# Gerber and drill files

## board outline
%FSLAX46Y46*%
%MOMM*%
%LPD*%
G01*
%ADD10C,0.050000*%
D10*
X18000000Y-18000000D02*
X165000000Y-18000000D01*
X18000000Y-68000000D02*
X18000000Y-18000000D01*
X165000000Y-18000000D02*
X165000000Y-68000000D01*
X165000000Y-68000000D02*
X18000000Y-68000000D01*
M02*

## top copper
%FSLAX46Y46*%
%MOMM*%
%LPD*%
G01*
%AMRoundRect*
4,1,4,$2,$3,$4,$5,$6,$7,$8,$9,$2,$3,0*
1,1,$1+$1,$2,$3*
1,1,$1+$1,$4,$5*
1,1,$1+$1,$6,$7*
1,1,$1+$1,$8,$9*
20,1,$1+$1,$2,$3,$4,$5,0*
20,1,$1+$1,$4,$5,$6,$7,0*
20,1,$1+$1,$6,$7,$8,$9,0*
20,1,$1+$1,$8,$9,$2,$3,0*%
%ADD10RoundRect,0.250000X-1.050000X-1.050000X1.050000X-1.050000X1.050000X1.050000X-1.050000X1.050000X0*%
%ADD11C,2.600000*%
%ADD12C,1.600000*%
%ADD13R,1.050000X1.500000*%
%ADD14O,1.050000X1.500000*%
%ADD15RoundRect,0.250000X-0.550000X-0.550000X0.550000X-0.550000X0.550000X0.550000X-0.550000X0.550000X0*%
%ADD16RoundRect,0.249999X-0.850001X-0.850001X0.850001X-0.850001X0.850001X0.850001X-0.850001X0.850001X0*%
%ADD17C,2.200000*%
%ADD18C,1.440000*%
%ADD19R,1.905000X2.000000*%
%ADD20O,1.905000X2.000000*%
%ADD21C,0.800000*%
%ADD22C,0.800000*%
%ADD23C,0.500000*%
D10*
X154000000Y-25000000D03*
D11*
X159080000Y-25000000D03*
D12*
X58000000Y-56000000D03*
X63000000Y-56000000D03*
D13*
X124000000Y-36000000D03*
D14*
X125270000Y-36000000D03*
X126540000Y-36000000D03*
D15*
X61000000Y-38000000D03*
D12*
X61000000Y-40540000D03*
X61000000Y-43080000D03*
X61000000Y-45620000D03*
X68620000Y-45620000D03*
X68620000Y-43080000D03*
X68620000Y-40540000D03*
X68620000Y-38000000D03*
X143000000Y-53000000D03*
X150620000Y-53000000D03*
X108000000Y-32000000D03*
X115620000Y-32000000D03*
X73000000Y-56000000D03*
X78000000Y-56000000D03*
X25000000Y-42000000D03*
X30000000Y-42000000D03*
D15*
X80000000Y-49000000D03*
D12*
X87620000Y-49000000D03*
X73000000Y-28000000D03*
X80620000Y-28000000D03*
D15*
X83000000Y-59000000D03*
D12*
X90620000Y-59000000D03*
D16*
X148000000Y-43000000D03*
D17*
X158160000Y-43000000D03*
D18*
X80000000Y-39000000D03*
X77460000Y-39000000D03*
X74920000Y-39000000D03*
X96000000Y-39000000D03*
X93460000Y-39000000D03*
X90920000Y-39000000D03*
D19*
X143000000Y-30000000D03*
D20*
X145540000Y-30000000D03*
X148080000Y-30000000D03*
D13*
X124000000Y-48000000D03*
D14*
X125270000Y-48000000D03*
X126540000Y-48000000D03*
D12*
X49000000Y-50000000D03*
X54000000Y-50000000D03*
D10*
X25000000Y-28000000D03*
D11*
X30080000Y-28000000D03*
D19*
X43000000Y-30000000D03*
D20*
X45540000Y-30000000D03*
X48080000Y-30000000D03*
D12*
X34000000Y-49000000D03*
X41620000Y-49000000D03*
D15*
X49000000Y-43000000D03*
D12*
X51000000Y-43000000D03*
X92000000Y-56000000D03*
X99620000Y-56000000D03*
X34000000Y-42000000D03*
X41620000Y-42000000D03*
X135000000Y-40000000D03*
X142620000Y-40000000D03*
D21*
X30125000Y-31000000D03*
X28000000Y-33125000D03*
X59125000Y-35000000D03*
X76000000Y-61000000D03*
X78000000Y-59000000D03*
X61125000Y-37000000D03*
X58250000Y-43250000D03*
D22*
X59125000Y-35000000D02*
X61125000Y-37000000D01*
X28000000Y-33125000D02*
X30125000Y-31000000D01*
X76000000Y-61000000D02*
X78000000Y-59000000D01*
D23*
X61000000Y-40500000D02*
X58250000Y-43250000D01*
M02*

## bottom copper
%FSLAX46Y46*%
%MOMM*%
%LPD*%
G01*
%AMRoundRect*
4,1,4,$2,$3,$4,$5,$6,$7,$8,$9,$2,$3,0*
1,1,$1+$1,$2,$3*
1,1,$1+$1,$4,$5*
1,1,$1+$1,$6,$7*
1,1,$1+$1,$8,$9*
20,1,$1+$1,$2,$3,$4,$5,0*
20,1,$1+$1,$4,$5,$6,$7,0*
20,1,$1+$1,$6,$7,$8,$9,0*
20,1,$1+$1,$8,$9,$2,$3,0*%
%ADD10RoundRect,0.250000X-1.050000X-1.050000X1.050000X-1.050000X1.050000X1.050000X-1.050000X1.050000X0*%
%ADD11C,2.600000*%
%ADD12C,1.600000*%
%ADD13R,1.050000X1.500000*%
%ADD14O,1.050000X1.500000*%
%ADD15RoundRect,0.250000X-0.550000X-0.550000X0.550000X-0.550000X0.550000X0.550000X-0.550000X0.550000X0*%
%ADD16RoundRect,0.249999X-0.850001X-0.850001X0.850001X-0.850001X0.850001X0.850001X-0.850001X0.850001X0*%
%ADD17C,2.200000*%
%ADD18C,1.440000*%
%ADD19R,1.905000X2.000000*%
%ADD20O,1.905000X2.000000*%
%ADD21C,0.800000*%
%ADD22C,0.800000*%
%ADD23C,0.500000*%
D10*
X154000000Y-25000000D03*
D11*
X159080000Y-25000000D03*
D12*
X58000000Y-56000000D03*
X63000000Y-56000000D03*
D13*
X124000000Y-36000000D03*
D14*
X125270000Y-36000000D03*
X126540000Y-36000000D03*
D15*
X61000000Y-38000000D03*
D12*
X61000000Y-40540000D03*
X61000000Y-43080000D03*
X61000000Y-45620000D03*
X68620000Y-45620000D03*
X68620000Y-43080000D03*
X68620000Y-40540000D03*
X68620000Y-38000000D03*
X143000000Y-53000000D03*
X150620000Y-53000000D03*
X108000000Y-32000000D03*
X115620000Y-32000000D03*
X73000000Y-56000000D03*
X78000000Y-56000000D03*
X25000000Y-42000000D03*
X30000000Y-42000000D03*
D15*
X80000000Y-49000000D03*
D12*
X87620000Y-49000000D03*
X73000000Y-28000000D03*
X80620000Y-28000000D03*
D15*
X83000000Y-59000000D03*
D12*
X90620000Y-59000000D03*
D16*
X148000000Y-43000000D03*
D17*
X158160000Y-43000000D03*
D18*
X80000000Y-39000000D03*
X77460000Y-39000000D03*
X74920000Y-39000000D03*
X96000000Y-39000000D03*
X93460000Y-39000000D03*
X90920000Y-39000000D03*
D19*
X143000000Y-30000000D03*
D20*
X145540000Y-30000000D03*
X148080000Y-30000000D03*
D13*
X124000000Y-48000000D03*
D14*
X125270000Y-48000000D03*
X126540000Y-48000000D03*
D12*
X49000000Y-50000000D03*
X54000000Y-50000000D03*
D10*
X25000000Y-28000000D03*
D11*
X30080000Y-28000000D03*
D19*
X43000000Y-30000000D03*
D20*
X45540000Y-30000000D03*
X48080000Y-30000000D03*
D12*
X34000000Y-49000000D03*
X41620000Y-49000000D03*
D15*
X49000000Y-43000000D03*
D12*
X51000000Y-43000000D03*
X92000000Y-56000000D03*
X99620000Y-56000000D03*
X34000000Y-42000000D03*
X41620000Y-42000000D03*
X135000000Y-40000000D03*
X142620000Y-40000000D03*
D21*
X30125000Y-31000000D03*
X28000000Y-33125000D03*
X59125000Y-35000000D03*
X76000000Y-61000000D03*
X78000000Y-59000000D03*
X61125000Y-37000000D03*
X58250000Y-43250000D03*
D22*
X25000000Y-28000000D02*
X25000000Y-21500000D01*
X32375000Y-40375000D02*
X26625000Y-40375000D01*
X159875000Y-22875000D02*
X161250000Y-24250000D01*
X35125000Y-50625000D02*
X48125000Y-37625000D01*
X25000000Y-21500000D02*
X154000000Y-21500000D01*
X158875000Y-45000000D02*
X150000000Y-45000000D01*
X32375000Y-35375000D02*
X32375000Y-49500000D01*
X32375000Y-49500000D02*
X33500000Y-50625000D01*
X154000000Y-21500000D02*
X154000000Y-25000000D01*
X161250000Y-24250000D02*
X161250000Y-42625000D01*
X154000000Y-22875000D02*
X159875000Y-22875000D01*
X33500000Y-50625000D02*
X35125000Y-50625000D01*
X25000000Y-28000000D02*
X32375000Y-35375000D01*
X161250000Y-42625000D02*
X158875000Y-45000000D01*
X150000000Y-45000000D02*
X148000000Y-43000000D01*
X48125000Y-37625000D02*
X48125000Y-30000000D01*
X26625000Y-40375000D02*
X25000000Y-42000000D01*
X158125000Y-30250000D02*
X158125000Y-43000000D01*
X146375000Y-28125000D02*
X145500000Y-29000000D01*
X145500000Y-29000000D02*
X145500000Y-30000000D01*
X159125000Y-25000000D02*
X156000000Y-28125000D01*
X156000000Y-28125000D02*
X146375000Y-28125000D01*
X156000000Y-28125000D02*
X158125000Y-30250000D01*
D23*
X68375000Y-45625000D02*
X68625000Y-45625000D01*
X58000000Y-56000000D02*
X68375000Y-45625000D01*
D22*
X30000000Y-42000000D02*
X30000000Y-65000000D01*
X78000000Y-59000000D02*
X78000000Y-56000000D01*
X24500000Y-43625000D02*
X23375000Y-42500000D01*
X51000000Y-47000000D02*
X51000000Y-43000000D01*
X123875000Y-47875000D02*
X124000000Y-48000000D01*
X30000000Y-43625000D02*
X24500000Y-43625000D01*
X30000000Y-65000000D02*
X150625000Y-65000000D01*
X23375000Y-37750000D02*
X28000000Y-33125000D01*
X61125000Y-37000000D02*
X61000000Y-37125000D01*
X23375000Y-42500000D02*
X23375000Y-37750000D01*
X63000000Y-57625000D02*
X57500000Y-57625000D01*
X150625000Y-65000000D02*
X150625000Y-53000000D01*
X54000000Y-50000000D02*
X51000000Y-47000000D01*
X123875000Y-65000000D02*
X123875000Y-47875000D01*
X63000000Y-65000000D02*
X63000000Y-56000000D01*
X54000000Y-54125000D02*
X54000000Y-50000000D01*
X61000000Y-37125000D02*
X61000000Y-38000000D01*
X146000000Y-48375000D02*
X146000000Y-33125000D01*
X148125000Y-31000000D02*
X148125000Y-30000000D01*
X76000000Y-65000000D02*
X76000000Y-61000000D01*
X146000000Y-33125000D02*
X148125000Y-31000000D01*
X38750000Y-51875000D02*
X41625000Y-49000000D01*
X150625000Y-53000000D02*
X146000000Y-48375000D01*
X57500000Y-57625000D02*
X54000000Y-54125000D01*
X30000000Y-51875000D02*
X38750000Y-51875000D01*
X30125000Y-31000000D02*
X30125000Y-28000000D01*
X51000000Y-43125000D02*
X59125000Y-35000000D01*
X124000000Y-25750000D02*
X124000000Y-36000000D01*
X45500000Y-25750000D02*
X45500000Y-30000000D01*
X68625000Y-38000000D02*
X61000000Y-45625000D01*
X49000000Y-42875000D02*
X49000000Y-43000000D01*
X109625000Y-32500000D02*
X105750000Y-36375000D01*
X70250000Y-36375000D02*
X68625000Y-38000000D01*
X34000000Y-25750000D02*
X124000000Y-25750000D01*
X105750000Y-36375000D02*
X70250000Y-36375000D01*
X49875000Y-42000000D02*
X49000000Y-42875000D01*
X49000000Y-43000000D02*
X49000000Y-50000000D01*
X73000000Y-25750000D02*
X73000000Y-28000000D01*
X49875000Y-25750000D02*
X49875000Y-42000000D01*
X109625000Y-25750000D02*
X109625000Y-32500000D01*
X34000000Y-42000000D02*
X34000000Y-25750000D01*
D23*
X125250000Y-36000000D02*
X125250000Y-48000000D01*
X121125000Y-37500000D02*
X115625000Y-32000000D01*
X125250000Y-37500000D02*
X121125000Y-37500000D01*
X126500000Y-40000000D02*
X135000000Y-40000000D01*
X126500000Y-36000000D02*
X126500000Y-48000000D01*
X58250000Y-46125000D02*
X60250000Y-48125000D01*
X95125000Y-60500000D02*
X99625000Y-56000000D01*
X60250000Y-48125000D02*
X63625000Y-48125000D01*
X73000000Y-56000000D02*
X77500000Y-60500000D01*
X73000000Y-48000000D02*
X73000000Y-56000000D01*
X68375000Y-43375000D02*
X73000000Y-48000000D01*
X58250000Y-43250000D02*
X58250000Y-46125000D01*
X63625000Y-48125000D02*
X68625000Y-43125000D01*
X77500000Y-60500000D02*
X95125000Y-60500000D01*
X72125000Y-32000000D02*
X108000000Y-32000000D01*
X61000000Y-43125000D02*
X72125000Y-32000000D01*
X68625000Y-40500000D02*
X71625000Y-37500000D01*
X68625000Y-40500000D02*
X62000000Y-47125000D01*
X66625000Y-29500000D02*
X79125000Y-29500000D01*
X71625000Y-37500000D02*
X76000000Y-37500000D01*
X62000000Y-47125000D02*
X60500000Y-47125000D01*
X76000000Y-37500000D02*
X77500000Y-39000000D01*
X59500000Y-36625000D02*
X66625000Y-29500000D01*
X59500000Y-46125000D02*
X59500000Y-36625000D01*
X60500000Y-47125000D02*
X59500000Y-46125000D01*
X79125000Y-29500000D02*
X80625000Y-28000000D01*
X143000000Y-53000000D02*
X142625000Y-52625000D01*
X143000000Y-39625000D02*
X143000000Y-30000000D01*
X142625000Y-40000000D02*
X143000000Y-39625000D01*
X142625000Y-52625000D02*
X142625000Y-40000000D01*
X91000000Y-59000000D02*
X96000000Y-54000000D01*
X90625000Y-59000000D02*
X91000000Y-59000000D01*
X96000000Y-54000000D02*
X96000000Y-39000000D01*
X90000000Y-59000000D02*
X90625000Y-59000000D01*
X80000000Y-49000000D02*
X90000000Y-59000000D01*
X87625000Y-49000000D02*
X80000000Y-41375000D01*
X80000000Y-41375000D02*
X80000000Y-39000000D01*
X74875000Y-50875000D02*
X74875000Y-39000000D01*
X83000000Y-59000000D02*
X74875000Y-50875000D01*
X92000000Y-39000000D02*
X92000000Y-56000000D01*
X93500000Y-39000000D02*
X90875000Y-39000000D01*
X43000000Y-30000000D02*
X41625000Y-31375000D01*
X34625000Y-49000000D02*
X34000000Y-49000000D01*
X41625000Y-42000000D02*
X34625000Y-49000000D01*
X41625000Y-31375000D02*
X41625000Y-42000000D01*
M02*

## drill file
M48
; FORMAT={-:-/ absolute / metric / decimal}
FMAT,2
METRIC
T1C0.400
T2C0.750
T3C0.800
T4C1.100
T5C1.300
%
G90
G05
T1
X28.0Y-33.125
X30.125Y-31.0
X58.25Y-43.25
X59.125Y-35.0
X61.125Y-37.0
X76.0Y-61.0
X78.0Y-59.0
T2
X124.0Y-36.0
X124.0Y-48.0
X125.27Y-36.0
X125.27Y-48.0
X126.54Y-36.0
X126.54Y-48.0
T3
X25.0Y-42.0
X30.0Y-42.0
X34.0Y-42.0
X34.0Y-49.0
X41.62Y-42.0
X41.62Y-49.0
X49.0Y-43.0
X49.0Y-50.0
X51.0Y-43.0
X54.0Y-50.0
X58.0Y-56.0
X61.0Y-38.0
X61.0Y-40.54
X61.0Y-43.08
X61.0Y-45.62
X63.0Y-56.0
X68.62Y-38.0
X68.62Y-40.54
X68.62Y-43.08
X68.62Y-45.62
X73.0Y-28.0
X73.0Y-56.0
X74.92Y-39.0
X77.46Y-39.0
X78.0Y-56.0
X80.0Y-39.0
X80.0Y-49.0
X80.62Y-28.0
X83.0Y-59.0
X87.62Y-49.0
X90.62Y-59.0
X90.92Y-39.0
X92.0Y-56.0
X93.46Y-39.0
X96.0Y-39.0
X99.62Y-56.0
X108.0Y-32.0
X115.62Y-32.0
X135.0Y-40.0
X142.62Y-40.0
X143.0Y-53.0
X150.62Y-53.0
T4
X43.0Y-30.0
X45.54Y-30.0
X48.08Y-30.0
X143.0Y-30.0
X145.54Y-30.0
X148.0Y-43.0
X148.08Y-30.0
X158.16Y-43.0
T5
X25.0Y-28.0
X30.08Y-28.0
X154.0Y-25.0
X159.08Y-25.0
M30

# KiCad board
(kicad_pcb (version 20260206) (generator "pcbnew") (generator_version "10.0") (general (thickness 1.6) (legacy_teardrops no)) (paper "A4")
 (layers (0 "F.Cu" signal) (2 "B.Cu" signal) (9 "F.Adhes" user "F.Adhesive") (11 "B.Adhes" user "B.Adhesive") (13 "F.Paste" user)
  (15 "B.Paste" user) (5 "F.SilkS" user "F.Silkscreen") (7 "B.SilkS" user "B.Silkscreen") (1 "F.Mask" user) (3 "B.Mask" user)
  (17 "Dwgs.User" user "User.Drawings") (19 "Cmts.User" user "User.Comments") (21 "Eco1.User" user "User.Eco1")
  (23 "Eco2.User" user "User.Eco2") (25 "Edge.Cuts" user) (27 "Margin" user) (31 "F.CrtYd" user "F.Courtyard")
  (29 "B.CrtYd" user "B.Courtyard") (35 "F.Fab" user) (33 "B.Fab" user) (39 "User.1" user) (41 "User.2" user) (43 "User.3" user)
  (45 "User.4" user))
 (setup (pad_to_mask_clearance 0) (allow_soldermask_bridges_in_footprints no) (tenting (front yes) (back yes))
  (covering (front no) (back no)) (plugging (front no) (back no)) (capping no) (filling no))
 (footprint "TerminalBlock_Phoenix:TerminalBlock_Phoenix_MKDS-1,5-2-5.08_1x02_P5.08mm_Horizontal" (layer "F.Cu") (at 154 25)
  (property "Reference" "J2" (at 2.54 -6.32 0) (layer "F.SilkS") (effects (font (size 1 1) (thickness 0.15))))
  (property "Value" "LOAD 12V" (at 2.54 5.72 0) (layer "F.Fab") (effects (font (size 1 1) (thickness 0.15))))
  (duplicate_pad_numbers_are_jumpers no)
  (pad "1" thru_hole roundrect (at 0 0) (size 2.6 2.6) (drill 1.3) (layers "*.Cu" "*.Mask") (remove_unused_layers no)
   (roundrect_rratio 0.096154) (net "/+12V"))
  (pad "2" thru_hole circle (at 5.08 0) (size 2.6 2.6) (drill 1.3) (layers "*.Cu" "*.Mask") (remove_unused_layers no) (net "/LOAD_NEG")))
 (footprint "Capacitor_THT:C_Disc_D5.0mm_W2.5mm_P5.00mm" (layer "F.Cu") (at 58 56)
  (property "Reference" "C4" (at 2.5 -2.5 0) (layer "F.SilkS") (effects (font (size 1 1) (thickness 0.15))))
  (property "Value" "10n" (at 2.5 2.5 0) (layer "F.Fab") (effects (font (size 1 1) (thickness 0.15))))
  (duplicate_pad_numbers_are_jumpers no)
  (pad "1" thru_hole circle (at 0 0) (size 1.6 1.6) (drill 0.8) (layers "*.Cu" "*.Mask") (remove_unused_layers no) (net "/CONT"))
  (pad "2" thru_hole circle (at 5 0) (size 1.6 1.6) (drill 0.8) (layers "*.Cu" "*.Mask") (remove_unused_layers no) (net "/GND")))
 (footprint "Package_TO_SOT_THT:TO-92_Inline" (layer "F.Cu") (at 124 36)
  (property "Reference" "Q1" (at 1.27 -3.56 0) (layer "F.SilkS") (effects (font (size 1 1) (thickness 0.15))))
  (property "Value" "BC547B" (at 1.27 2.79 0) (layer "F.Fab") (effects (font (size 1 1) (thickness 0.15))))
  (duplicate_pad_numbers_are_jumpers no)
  (pad "1" thru_hole rect (at 0 0) (size 1.05 1.5) (drill 0.75) (layers "*.Cu" "*.Mask") (remove_unused_layers no) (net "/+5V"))
  (pad "2" thru_hole oval (at 1.27 0) (size 1.05 1.5) (drill 0.75) (layers "*.Cu" "*.Mask") (remove_unused_layers no) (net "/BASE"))
  (pad "3" thru_hole oval (at 2.54 0) (size 1.05 1.5) (drill 0.75) (layers "*.Cu" "*.Mask") (remove_unused_layers no) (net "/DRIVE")))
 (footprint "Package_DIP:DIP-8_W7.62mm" (layer "F.Cu") (at 61 38)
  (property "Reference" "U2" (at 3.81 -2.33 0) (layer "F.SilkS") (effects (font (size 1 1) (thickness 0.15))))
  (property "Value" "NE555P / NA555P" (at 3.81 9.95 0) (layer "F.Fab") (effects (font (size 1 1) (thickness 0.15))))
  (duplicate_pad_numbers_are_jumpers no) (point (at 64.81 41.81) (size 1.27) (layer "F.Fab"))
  (pad "1" thru_hole roundrect (at 0 0) (size 1.6 1.6) (drill 0.8) (layers "*.Cu" "*.Mask") (remove_unused_layers no)
   (roundrect_rratio 0.15625) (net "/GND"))
  (pad "2" thru_hole circle (at 0 2.54) (size 1.6 1.6) (drill 0.8) (layers "*.Cu" "*.Mask") (remove_unused_layers no) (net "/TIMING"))
  (pad "3" thru_hole circle (at 0 5.08) (size 1.6 1.6) (drill 0.8) (layers "*.Cu" "*.Mask") (remove_unused_layers no) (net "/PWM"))
  (pad "4" thru_hole circle (at 0 7.62) (size 1.6 1.6) (drill 0.8) (layers "*.Cu" "*.Mask") (remove_unused_layers no) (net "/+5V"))
  (pad "5" thru_hole circle (at 7.62 7.62) (size 1.6 1.6) (drill 0.8) (layers "*.Cu" "*.Mask") (remove_unused_layers no) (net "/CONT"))
  (pad "6" thru_hole circle (at 7.62 5.08) (size 1.6 1.6) (drill 0.8) (layers "*.Cu" "*.Mask") (remove_unused_layers no) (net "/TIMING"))
  (pad "7" thru_hole circle (at 7.62 2.54) (size 1.6 1.6) (drill 0.8) (layers "*.Cu" "*.Mask") (remove_unused_layers no) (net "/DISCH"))
  (pad "8" thru_hole circle (at 7.62 0) (size 1.6 1.6) (drill 0.8) (layers "*.Cu" "*.Mask") (remove_unused_layers no) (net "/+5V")))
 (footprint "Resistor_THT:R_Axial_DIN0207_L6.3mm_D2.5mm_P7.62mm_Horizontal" (layer "F.Cu") (at 143 53)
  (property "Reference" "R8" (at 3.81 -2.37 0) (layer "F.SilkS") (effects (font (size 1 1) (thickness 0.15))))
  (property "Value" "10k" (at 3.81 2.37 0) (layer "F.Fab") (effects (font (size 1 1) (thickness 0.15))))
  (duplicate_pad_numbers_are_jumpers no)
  (pad "1" thru_hole circle (at 0 0) (size 1.6 1.6) (drill 0.8) (layers "*.Cu" "*.Mask") (remove_unused_layers no) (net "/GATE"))
  (pad "2" thru_hole circle (at 7.62 0) (size 1.6 1.6) (drill 0.8) (layers "*.Cu" "*.Mask") (remove_unused_layers no) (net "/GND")))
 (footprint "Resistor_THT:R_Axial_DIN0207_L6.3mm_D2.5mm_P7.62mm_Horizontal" (layer "F.Cu") (at 108 32)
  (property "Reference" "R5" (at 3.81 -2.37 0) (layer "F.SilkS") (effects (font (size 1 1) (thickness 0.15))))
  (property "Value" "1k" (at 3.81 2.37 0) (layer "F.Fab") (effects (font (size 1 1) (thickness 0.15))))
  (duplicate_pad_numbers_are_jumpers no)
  (pad "1" thru_hole circle (at 0 0) (size 1.6 1.6) (drill 0.8) (layers "*.Cu" "*.Mask") (remove_unused_layers no) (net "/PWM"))
  (pad "2" thru_hole circle (at 7.62 0) (size 1.6 1.6) (drill 0.8) (layers "*.Cu" "*.Mask") (remove_unused_layers no) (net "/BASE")))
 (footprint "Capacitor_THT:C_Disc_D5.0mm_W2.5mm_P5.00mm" (layer "F.Cu") (at 73 56)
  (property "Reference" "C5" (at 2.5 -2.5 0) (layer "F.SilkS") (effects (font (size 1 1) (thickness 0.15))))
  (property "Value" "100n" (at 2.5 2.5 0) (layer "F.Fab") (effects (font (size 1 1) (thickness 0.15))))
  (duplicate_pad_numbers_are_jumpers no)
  (pad "1" thru_hole circle (at 0 0) (size 1.6 1.6) (drill 0.8) (layers "*.Cu" "*.Mask") (remove_unused_layers no) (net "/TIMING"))
  (pad "2" thru_hole circle (at 5 0) (size 1.6 1.6) (drill 0.8) (layers "*.Cu" "*.Mask") (remove_unused_layers no) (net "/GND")))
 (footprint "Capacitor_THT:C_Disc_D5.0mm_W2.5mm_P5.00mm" (layer "F.Cu") (at 25 42)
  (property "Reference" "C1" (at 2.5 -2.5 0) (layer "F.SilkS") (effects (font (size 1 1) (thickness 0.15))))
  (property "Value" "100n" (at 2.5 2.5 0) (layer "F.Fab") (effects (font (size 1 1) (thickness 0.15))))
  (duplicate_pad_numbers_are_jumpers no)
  (pad "1" thru_hole circle (at 0 0) (size 1.6 1.6) (drill 0.8) (layers "*.Cu" "*.Mask") (remove_unused_layers no) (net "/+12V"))
  (pad "2" thru_hole circle (at 5 0) (size 1.6 1.6) (drill 0.8) (layers "*.Cu" "*.Mask") (remove_unused_layers no) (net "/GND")))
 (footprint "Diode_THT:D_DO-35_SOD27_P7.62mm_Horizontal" (layer "F.Cu") (at 80 49)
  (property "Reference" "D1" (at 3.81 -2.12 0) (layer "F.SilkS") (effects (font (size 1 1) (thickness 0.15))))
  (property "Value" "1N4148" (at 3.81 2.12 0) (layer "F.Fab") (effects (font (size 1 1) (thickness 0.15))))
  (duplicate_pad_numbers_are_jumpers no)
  (pad "1" thru_hole roundrect (at 0 0) (size 1.6 1.6) (drill 0.8) (layers "*.Cu" "*.Mask") (remove_unused_layers no)
   (roundrect_rratio 0.15625) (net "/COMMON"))
  (pad "2" thru_hole circle (at 7.62 0) (size 1.6 1.6) (drill 0.8) (layers "*.Cu" "*.Mask") (remove_unused_layers no) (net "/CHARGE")))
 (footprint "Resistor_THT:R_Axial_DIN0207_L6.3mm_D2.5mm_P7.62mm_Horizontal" (layer "F.Cu") (at 73 28)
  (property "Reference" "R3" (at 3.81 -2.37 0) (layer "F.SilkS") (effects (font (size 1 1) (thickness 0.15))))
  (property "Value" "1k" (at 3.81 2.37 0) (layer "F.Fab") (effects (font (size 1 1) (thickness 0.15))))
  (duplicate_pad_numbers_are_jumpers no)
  (pad "1" thru_hole circle (at 0 0) (size 1.6 1.6) (drill 0.8) (layers "*.Cu" "*.Mask") (remove_unused_layers no) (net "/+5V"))
  (pad "2" thru_hole circle (at 7.62 0) (size 1.6 1.6) (drill 0.8) (layers "*.Cu" "*.Mask") (remove_unused_layers no) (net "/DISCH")))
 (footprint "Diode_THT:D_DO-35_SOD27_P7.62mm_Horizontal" (layer "F.Cu") (at 83 59)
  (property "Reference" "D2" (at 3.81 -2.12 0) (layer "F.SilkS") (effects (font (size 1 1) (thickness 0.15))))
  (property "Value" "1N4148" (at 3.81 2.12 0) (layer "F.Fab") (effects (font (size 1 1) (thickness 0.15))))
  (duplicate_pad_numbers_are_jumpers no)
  (pad "1" thru_hole roundrect (at 0 0) (size 1.6 1.6) (drill 0.8) (layers "*.Cu" "*.Mask") (remove_unused_layers no)
   (roundrect_rratio 0.15625) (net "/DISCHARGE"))
  (pad "2" thru_hole circle (at 7.62 0) (size 1.6 1.6) (drill 0.8) (layers "*.Cu" "*.Mask") (remove_unused_layers no) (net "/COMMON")))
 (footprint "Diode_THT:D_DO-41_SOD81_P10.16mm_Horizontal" (layer "F.Cu") (at 148 43)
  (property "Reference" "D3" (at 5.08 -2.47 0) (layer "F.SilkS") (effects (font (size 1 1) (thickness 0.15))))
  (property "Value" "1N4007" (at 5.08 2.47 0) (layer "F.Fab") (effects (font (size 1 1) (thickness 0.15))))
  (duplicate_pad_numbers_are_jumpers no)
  (pad "1" thru_hole roundrect (at 0 0) (size 2.2 2.2) (drill 1.1) (layers "*.Cu" "*.Mask") (remove_unused_layers no)
   (roundrect_rratio 0.113636) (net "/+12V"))
  (pad "2" thru_hole circle (at 10.16 0) (size 2.2 2.2) (drill 1.1) (layers "*.Cu" "*.Mask") (remove_unused_layers no) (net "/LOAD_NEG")))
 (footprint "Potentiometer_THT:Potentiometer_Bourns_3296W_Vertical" (layer "F.Cu") (at 80 39)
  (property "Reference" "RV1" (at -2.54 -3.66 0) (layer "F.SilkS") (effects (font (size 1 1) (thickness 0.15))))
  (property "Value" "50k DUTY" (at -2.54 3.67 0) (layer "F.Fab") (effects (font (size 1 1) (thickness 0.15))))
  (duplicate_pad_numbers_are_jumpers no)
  (pad "1" thru_hole circle (at 0 0) (size 1.44 1.44) (drill 0.8) (layers "*.Cu" "*.Mask") (remove_unused_layers no) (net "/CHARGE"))
  (pad "2" thru_hole circle (at -2.54 0) (size 1.44 1.44) (drill 0.8) (layers "*.Cu" "*.Mask") (remove_unused_layers no) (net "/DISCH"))
  (pad "3" thru_hole circle (at -5.08 0) (size 1.44 1.44) (drill 0.8) (layers "*.Cu" "*.Mask") (remove_unused_layers no) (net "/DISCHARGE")))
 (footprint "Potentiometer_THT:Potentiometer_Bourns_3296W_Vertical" (layer "F.Cu") (at 96 39)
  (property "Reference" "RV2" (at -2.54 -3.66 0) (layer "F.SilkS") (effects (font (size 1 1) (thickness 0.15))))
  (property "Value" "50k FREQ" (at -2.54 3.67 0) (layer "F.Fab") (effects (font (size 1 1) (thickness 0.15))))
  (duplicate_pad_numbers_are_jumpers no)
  (pad "1" thru_hole circle (at 0 0) (size 1.44 1.44) (drill 0.8) (layers "*.Cu" "*.Mask") (remove_unused_layers no) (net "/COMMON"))
  (pad "2" thru_hole circle (at -2.54 0) (size 1.44 1.44) (drill 0.8) (layers "*.Cu" "*.Mask") (remove_unused_layers no) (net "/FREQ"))
  (pad "3" thru_hole circle (at -5.08 0) (size 1.44 1.44) (drill 0.8) (layers "*.Cu" "*.Mask") (remove_unused_layers no) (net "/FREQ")))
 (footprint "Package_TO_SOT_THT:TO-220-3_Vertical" (layer "F.Cu") (at 143 30)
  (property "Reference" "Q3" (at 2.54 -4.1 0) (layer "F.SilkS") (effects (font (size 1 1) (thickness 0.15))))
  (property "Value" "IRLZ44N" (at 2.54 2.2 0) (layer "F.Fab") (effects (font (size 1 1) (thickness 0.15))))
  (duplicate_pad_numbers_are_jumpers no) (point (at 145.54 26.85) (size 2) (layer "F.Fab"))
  (pad "1" thru_hole rect (at 0 0) (size 1.905 2) (drill 1.1) (layers "*.Cu" "*.Mask") (remove_unused_layers no) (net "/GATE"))
  (pad "2" thru_hole oval (at 2.54 0) (size 1.905 2) (drill 1.1) (layers "*.Cu" "*.Mask") (remove_unused_layers no) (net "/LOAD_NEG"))
  (pad "3" thru_hole oval (at 5.08 0) (size 1.905 2) (drill 1.1) (layers "*.Cu" "*.Mask") (remove_unused_layers no) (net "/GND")))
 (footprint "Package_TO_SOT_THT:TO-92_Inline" (layer "F.Cu") (at 124 48)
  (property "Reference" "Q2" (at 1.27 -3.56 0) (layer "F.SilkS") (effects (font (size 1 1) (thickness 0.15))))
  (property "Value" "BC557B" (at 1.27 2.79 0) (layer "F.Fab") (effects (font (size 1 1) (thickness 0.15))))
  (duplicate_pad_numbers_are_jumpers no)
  (pad "1" thru_hole rect (at 0 0) (size 1.05 1.5) (drill 0.75) (layers "*.Cu" "*.Mask") (remove_unused_layers no) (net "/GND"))
  (pad "2" thru_hole oval (at 1.27 0) (size 1.05 1.5) (drill 0.75) (layers "*.Cu" "*.Mask") (remove_unused_layers no) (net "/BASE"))
  (pad "3" thru_hole oval (at 2.54 0) (size 1.05 1.5) (drill 0.75) (layers "*.Cu" "*.Mask") (remove_unused_layers no) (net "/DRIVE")))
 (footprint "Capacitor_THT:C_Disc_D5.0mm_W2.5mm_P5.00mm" (layer "F.Cu") (at 49 50)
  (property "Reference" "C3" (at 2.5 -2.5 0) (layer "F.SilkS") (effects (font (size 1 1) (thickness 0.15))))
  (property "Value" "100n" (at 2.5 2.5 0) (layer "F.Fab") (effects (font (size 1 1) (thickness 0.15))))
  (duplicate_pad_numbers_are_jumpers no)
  (pad "1" thru_hole circle (at 0 0) (size 1.6 1.6) (drill 0.8) (layers "*.Cu" "*.Mask") (remove_unused_layers no) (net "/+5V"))
  (pad "2" thru_hole circle (at 5 0) (size 1.6 1.6) (drill 0.8) (layers "*.Cu" "*.Mask") (remove_unused_layers no) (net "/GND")))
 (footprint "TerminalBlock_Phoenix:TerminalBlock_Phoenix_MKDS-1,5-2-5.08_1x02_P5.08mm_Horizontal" (layer "F.Cu") (at 25 28)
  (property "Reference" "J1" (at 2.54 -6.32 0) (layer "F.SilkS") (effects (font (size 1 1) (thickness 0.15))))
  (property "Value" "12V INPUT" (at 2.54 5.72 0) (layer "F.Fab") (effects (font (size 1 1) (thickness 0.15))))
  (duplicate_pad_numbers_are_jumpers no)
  (pad "1" thru_hole roundrect (at 0 0) (size 2.6 2.6) (drill 1.3) (layers "*.Cu" "*.Mask") (remove_unused_layers no)
   (roundrect_rratio 0.096154) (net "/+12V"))
  (pad "2" thru_hole circle (at 5.08 0) (size 2.6 2.6) (drill 1.3) (layers "*.Cu" "*.Mask") (remove_unused_layers no) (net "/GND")))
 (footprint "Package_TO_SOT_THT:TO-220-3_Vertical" (layer "F.Cu") (at 43 30)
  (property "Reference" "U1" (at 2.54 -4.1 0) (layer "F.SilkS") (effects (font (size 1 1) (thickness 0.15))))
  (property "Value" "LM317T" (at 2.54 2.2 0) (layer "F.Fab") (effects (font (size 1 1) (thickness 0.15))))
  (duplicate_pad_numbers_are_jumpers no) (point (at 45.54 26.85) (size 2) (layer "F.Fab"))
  (pad "1" thru_hole rect (at 0 0) (size 1.905 2) (drill 1.1) (layers "*.Cu" "*.Mask") (remove_unused_layers no) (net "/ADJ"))
  (pad "2" thru_hole oval (at 2.54 0) (size 1.905 2) (drill 1.1) (layers "*.Cu" "*.Mask") (remove_unused_layers no) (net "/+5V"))
  (pad "3" thru_hole oval (at 5.08 0) (size 1.905 2) (drill 1.1) (layers "*.Cu" "*.Mask") (remove_unused_layers no) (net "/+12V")))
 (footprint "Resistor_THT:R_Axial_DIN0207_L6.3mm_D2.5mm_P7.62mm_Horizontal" (layer "F.Cu") (at 34 49)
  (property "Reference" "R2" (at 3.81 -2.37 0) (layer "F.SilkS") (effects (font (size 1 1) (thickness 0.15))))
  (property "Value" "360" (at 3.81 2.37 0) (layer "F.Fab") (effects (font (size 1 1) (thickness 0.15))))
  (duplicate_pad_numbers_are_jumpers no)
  (pad "1" thru_hole circle (at 0 0) (size 1.6 1.6) (drill 0.8) (layers "*.Cu" "*.Mask") (remove_unused_layers no) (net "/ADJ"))
  (pad "2" thru_hole circle (at 7.62 0) (size 1.6 1.6) (drill 0.8) (layers "*.Cu" "*.Mask") (remove_unused_layers no) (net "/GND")))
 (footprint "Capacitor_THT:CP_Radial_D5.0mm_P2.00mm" (layer "F.Cu") (at 49 43)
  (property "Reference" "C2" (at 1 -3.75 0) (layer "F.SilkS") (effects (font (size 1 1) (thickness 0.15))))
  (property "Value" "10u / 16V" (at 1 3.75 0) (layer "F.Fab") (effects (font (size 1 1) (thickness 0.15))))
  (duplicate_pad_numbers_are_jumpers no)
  (pad "1" thru_hole roundrect (at 0 0) (size 1.6 1.6) (drill 0.8) (layers "*.Cu" "*.Mask") (remove_unused_layers no)
   (roundrect_rratio 0.15625) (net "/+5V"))
  (pad "2" thru_hole circle (at 2 0) (size 1.6 1.6) (drill 0.8) (layers "*.Cu" "*.Mask") (remove_unused_layers no) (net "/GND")))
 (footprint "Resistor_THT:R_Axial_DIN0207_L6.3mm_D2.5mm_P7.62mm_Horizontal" (layer "F.Cu") (at 92 56)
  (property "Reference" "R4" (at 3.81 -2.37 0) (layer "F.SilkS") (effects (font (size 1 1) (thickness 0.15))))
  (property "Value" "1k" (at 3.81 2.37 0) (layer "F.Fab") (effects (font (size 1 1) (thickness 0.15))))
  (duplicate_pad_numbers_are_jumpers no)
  (pad "1" thru_hole circle (at 0 0) (size 1.6 1.6) (drill 0.8) (layers "*.Cu" "*.Mask") (remove_unused_layers no) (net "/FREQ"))
  (pad "2" thru_hole circle (at 7.62 0) (size 1.6 1.6) (drill 0.8) (layers "*.Cu" "*.Mask") (remove_unused_layers no) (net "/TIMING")))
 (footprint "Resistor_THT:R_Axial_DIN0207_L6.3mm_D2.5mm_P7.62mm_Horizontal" (layer "F.Cu") (at 34 42)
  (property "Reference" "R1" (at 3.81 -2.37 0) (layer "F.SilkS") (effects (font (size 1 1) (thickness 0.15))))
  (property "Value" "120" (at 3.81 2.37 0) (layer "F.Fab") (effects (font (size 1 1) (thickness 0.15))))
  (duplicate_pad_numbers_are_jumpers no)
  (pad "1" thru_hole circle (at 0 0) (size 1.6 1.6) (drill 0.8) (layers "*.Cu" "*.Mask") (remove_unused_layers no) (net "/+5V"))
  (pad "2" thru_hole circle (at 7.62 0) (size 1.6 1.6) (drill 0.8) (layers "*.Cu" "*.Mask") (remove_unused_layers no) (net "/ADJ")))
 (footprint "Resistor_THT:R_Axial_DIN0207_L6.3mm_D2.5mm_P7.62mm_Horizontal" (layer "F.Cu") (at 135 40)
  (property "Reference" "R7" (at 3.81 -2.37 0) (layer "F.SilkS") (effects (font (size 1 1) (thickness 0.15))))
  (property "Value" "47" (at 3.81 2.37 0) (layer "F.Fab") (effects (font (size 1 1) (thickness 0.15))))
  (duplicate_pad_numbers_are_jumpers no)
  (pad "1" thru_hole circle (at 0 0) (size 1.6 1.6) (drill 0.8) (layers "*.Cu" "*.Mask") (remove_unused_layers no) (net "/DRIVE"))
  (pad "2" thru_hole circle (at 7.62 0) (size 1.6 1.6) (drill 0.8) (layers "*.Cu" "*.Mask") (remove_unused_layers no) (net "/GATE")))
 (gr_line (start 18 18) (end 165 18) (stroke (width 0.05) (type default)) (layer "Edge.Cuts"))
 (gr_line (start 18 68) (end 18 18) (stroke (width 0.05) (type default)) (layer "Edge.Cuts"))
 (gr_line (start 165 18) (end 165 68) (stroke (width 0.05) (type default)) (layer "Edge.Cuts"))
 (gr_line (start 165 68) (end 18 68) (stroke (width 0.05) (type default)) (layer "Edge.Cuts"))
 (segment (start 25 28) (end 25 21.5) (width 0.8) (layer "B.Cu") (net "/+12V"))
 (segment (start 32.375 40.375) (end 26.625 40.375) (width 0.8) (layer "B.Cu") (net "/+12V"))
 (segment (start 159.875 22.875) (end 161.25 24.25) (width 0.8) (layer "B.Cu") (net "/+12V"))
 (segment (start 35.125 50.625) (end 48.125 37.625) (width 0.8) (layer "B.Cu") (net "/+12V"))
 (segment (start 25 21.5) (end 154 21.5) (width 0.8) (layer "B.Cu") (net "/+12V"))
 (segment (start 158.875 45) (end 150 45) (width 0.8) (layer "B.Cu") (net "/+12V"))
 (segment (start 32.375 35.375) (end 32.375 49.5) (width 0.8) (layer "B.Cu") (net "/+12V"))
 (segment (start 32.375 49.5) (end 33.5 50.625) (width 0.8) (layer "B.Cu") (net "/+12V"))
 (segment (start 154 21.5) (end 154 25) (width 0.8) (layer "B.Cu") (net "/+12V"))
 (segment (start 161.25 24.25) (end 161.25 42.625) (width 0.8) (layer "B.Cu") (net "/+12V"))
 (segment (start 154 22.875) (end 159.875 22.875) (width 0.8) (layer "B.Cu") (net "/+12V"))
 (segment (start 33.5 50.625) (end 35.125 50.625) (width 0.8) (layer "B.Cu") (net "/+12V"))
 (segment (start 25 28) (end 32.375 35.375) (width 0.8) (layer "B.Cu") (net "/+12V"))
 (segment (start 161.25 42.625) (end 158.875 45) (width 0.8) (layer "B.Cu") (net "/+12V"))
 (segment (start 150 45) (end 148 43) (width 0.8) (layer "B.Cu") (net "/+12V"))
 (segment (start 48.125 37.625) (end 48.125 30) (width 0.8) (layer "B.Cu") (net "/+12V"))
 (segment (start 26.625 40.375) (end 25 42) (width 0.8) (layer "B.Cu") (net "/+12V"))
 (segment (start 158.125 30.25) (end 158.125 43) (width 0.8) (layer "B.Cu") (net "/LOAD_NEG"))
 (segment (start 146.375 28.125) (end 145.5 29) (width 0.8) (layer "B.Cu") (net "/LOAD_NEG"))
 (segment (start 145.5 29) (end 145.5 30) (width 0.8) (layer "B.Cu") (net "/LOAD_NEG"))
 (segment (start 159.125 25) (end 156 28.125) (width 0.8) (layer "B.Cu") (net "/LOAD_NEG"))
 (segment (start 156 28.125) (end 146.375 28.125) (width 0.8) (layer "B.Cu") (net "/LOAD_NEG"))
 (segment (start 156 28.125) (end 158.125 30.25) (width 0.8) (layer "B.Cu") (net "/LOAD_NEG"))
 (segment (start 68.375 45.625) (end 68.625 45.625) (width 0.5) (layer "B.Cu") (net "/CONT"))
 (segment (start 58 56) (end 68.375 45.625) (width 0.5) (layer "B.Cu") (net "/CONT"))
 (segment (start 59.125 35) (end 61.125 37) (width 0.8) (layer "F.Cu") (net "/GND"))
 (segment (start 28 33.125) (end 30.125 31) (width 0.8) (layer "F.Cu") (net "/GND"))
 (segment (start 76 61) (end 78 59) (width 0.8) (layer "F.Cu") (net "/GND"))
 (via (at 30.125 31) (size 0.8) (drill 0.4) (layers "F.Cu" "B.Cu") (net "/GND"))
 (via (at 28 33.125) (size 0.8) (drill 0.4) (layers "F.Cu" "B.Cu") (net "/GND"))
 (via (at 59.125 35) (size 0.8) (drill 0.4) (layers "F.Cu" "B.Cu") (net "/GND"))
 (via (at 76 61) (size 0.8) (drill 0.4) (layers "F.Cu" "B.Cu") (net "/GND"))
 (via (at 78 59) (size 0.8) (drill 0.4) (layers "F.Cu" "B.Cu") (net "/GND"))
 (via (at 61.125 37) (size 0.8) (drill 0.4) (layers "F.Cu" "B.Cu") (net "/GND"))
 (segment (start 30 42) (end 30 65) (width 0.8) (layer "B.Cu") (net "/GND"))
 (segment (start 78 59) (end 78 56) (width 0.8) (layer "B.Cu") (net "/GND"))
 (segment (start 24.5 43.625) (end 23.375 42.5) (width 0.8) (layer "B.Cu") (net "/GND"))
 (segment (start 51 47) (end 51 43) (width 0.8) (layer "B.Cu") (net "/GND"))
 (segment (start 123.875 47.875) (end 124 48) (width 0.8) (layer "B.Cu") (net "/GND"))
 (segment (start 30 43.625) (end 24.5 43.625) (width 0.8) (layer "B.Cu") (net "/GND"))
 (segment (start 30 65) (end 150.625 65) (width 0.8) (layer "B.Cu") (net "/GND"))
 (segment (start 23.375 37.75) (end 28 33.125) (width 0.8) (layer "B.Cu") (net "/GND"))
 (segment (start 61.125 37) (end 61 37.125) (width 0.8) (layer "B.Cu") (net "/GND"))
 (segment (start 23.375 42.5) (end 23.375 37.75) (width 0.8) (layer "B.Cu") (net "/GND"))
 (segment (start 63 57.625) (end 57.5 57.625) (width 0.8) (layer "B.Cu") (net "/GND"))
 (segment (start 150.625 65) (end 150.625 53) (width 0.8) (layer "B.Cu") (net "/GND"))
 (segment (start 54 50) (end 51 47) (width 0.8) (layer "B.Cu") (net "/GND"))
 (segment (start 123.875 65) (end 123.875 47.875) (width 0.8) (layer "B.Cu") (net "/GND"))
 (segment (start 63 65) (end 63 56) (width 0.8) (layer "B.Cu") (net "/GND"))
 (segment (start 54 54.125) (end 54 50) (width 0.8) (layer "B.Cu") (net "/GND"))
 (segment (start 61 37.125) (end 61 38) (width 0.8) (layer "B.Cu") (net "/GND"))
 (segment (start 146 48.375) (end 146 33.125) (width 0.8) (layer "B.Cu") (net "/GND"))
 (segment (start 148.125 31) (end 148.125 30) (width 0.8) (layer "B.Cu") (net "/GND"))
 (segment (start 76 65) (end 76 61) (width 0.8) (layer "B.Cu") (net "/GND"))
 (segment (start 146 33.125) (end 148.125 31) (width 0.8) (layer "B.Cu") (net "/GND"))
 (segment (start 38.75 51.875) (end 41.625 49) (width 0.8) (layer "B.Cu") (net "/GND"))
 (segment (start 150.625 53) (end 146 48.375) (width 0.8) (layer "B.Cu") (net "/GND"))
 (segment (start 57.5 57.625) (end 54 54.125) (width 0.8) (layer "B.Cu") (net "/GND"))
 (segment (start 30 51.875) (end 38.75 51.875) (width 0.8) (layer "B.Cu") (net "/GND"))
 (segment (start 30.125 31) (end 30.125 28) (width 0.8) (layer "B.Cu") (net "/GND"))
 (segment (start 51 43.125) (end 59.125 35) (width 0.8) (layer "B.Cu") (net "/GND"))
 (segment (start 124 25.75) (end 124 36) (width 0.8) (layer "B.Cu") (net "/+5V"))
 (segment (start 45.5 25.75) (end 45.5 30) (width 0.8) (layer "B.Cu") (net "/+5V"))
 (segment (start 68.625 38) (end 61 45.625) (width 0.8) (layer "B.Cu") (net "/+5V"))
 (segment (start 49 42.875) (end 49 43) (width 0.8) (layer "B.Cu") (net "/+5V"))
 (segment (start 109.625 32.5) (end 105.75 36.375) (width 0.8) (layer "B.Cu") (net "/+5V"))
 (segment (start 70.25 36.375) (end 68.625 38) (width 0.8) (layer "B.Cu") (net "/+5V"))
 (segment (start 34 25.75) (end 124 25.75) (width 0.8) (layer "B.Cu") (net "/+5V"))
 (segment (start 105.75 36.375) (end 70.25 36.375) (width 0.8) (layer "B.Cu") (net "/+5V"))
 (segment (start 49.875 42) (end 49 42.875) (width 0.8) (layer "B.Cu") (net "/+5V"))
 (segment (start 49 43) (end 49 50) (width 0.8) (layer "B.Cu") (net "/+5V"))
 (segment (start 73 25.75) (end 73 28) (width 0.8) (layer "B.Cu") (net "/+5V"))
 (segment (start 49.875 25.75) (end 49.875 42) (width 0.8) (layer "B.Cu") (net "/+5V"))
 (segment (start 109.625 25.75) (end 109.625 32.5) (width 0.8) (layer "B.Cu") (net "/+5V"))
 (segment (start 34 42) (end 34 25.75) (width 0.8) (layer "B.Cu") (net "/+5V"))
 (segment (start 125.25 36) (end 125.25 48) (width 0.5) (layer "B.Cu") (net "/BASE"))
 (segment (start 121.125 37.5) (end 115.625 32) (width 0.5) (layer "B.Cu") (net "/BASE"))
 (segment (start 125.25 37.5) (end 121.125 37.5) (width 0.5) (layer "B.Cu") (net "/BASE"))
 (segment (start 126.5 40) (end 135 40) (width 0.5) (layer "B.Cu") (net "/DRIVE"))
 (segment (start 126.5 36) (end 126.5 48) (width 0.5) (layer "B.Cu") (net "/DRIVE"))
 (segment (start 61 40.5) (end 58.25 43.25) (width 0.5) (layer "F.Cu") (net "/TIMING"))
 (via (at 58.25 43.25) (size 0.8) (drill 0.4) (layers "F.Cu" "B.Cu") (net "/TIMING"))
 (segment (start 58.25 46.125) (end 60.25 48.125) (width 0.5) (layer "B.Cu") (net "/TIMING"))
 (segment (start 95.125 60.5) (end 99.625 56) (width 0.5) (layer "B.Cu") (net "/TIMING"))
 (segment (start 60.25 48.125) (end 63.625 48.125) (width 0.5) (layer "B.Cu") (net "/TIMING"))
 (segment (start 73 56) (end 77.5 60.5) (width 0.5) (layer "B.Cu") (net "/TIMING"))
 (segment (start 73 48) (end 73 56) (width 0.5) (layer "B.Cu") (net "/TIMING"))
 (segment (start 68.375 43.375) (end 73 48) (width 0.5) (layer "B.Cu") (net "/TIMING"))
 (segment (start 58.25 43.25) (end 58.25 46.125) (width 0.5) (layer "B.Cu") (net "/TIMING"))
 (segment (start 63.625 48.125) (end 68.625 43.125) (width 0.5) (layer "B.Cu") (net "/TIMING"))
 (segment (start 77.5 60.5) (end 95.125 60.5) (width 0.5) (layer "B.Cu") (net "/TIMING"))
 (segment (start 72.125 32) (end 108 32) (width 0.5) (layer "B.Cu") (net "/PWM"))
 (segment (start 61 43.125) (end 72.125 32) (width 0.5) (layer "B.Cu") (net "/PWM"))
 (segment (start 68.625 40.5) (end 71.625 37.5) (width 0.5) (layer "B.Cu") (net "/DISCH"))
 (segment (start 68.625 40.5) (end 62 47.125) (width 0.5) (layer "B.Cu") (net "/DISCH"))
 (segment (start 66.625 29.5) (end 79.125 29.5) (width 0.5) (layer "B.Cu") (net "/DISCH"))
 (segment (start 71.625 37.5) (end 76 37.5) (width 0.5) (layer "B.Cu") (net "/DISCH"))
 (segment (start 62 47.125) (end 60.5 47.125) (width 0.5) (layer "B.Cu") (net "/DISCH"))
 (segment (start 76 37.5) (end 77.5 39) (width 0.5) (layer "B.Cu") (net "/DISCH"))
 (segment (start 59.5 36.625) (end 66.625 29.5) (width 0.5) (layer "B.Cu") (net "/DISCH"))
 (segment (start 59.5 46.125) (end 59.5 36.625) (width 0.5) (layer "B.Cu") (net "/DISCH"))
 (segment (start 60.5 47.125) (end 59.5 46.125) (width 0.5) (layer "B.Cu") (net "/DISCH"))
 (segment (start 79.125 29.5) (end 80.625 28) (width 0.5) (layer "B.Cu") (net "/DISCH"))
 (segment (start 143 53) (end 142.625 52.625) (width 0.5) (layer "B.Cu") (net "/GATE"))
 (segment (start 143 39.625) (end 143 30) (width 0.5) (layer "B.Cu") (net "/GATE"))
 (segment (start 142.625 40) (end 143 39.625) (width 0.5) (layer "B.Cu") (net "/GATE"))
 (segment (start 142.625 52.625) (end 142.625 40) (width 0.5) (layer "B.Cu") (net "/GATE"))
 (segment (start 91 59) (end 96 54) (width 0.5) (layer "B.Cu") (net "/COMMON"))
 (segment (start 90.625 59) (end 91 59) (width 0.5) (layer "B.Cu") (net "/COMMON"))
 (segment (start 96 54) (end 96 39) (width 0.5) (layer "B.Cu") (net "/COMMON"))
 (segment (start 90 59) (end 90.625 59) (width 0.5) (layer "B.Cu") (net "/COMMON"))
 (segment (start 80 49) (end 90 59) (width 0.5) (layer "B.Cu") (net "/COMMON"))
 (segment (start 87.625 49) (end 80 41.375) (width 0.5) (layer "B.Cu") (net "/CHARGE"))
 (segment (start 80 41.375) (end 80 39) (width 0.5) (layer "B.Cu") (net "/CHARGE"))
 (segment (start 74.875 50.875) (end 74.875 39) (width 0.5) (layer "B.Cu") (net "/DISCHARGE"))
 (segment (start 83 59) (end 74.875 50.875) (width 0.5) (layer "B.Cu") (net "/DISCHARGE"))
 (segment (start 92 39) (end 92 56) (width 0.5) (layer "B.Cu") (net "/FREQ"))
 (segment (start 93.5 39) (end 90.875 39) (width 0.5) (layer "B.Cu") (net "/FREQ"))
 (segment (start 43 30) (end 41.625 31.375) (width 0.5) (layer "B.Cu") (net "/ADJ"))
 (segment (start 34.625 49) (end 34 49) (width 0.5) (layer "B.Cu") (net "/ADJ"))
 (segment (start 41.625 42) (end 34.625 49) (width 0.5) (layer "B.Cu") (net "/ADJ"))
 (segment (start 41.625 31.375) (end 41.625 42) (width 0.5) (layer "B.Cu") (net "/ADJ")))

